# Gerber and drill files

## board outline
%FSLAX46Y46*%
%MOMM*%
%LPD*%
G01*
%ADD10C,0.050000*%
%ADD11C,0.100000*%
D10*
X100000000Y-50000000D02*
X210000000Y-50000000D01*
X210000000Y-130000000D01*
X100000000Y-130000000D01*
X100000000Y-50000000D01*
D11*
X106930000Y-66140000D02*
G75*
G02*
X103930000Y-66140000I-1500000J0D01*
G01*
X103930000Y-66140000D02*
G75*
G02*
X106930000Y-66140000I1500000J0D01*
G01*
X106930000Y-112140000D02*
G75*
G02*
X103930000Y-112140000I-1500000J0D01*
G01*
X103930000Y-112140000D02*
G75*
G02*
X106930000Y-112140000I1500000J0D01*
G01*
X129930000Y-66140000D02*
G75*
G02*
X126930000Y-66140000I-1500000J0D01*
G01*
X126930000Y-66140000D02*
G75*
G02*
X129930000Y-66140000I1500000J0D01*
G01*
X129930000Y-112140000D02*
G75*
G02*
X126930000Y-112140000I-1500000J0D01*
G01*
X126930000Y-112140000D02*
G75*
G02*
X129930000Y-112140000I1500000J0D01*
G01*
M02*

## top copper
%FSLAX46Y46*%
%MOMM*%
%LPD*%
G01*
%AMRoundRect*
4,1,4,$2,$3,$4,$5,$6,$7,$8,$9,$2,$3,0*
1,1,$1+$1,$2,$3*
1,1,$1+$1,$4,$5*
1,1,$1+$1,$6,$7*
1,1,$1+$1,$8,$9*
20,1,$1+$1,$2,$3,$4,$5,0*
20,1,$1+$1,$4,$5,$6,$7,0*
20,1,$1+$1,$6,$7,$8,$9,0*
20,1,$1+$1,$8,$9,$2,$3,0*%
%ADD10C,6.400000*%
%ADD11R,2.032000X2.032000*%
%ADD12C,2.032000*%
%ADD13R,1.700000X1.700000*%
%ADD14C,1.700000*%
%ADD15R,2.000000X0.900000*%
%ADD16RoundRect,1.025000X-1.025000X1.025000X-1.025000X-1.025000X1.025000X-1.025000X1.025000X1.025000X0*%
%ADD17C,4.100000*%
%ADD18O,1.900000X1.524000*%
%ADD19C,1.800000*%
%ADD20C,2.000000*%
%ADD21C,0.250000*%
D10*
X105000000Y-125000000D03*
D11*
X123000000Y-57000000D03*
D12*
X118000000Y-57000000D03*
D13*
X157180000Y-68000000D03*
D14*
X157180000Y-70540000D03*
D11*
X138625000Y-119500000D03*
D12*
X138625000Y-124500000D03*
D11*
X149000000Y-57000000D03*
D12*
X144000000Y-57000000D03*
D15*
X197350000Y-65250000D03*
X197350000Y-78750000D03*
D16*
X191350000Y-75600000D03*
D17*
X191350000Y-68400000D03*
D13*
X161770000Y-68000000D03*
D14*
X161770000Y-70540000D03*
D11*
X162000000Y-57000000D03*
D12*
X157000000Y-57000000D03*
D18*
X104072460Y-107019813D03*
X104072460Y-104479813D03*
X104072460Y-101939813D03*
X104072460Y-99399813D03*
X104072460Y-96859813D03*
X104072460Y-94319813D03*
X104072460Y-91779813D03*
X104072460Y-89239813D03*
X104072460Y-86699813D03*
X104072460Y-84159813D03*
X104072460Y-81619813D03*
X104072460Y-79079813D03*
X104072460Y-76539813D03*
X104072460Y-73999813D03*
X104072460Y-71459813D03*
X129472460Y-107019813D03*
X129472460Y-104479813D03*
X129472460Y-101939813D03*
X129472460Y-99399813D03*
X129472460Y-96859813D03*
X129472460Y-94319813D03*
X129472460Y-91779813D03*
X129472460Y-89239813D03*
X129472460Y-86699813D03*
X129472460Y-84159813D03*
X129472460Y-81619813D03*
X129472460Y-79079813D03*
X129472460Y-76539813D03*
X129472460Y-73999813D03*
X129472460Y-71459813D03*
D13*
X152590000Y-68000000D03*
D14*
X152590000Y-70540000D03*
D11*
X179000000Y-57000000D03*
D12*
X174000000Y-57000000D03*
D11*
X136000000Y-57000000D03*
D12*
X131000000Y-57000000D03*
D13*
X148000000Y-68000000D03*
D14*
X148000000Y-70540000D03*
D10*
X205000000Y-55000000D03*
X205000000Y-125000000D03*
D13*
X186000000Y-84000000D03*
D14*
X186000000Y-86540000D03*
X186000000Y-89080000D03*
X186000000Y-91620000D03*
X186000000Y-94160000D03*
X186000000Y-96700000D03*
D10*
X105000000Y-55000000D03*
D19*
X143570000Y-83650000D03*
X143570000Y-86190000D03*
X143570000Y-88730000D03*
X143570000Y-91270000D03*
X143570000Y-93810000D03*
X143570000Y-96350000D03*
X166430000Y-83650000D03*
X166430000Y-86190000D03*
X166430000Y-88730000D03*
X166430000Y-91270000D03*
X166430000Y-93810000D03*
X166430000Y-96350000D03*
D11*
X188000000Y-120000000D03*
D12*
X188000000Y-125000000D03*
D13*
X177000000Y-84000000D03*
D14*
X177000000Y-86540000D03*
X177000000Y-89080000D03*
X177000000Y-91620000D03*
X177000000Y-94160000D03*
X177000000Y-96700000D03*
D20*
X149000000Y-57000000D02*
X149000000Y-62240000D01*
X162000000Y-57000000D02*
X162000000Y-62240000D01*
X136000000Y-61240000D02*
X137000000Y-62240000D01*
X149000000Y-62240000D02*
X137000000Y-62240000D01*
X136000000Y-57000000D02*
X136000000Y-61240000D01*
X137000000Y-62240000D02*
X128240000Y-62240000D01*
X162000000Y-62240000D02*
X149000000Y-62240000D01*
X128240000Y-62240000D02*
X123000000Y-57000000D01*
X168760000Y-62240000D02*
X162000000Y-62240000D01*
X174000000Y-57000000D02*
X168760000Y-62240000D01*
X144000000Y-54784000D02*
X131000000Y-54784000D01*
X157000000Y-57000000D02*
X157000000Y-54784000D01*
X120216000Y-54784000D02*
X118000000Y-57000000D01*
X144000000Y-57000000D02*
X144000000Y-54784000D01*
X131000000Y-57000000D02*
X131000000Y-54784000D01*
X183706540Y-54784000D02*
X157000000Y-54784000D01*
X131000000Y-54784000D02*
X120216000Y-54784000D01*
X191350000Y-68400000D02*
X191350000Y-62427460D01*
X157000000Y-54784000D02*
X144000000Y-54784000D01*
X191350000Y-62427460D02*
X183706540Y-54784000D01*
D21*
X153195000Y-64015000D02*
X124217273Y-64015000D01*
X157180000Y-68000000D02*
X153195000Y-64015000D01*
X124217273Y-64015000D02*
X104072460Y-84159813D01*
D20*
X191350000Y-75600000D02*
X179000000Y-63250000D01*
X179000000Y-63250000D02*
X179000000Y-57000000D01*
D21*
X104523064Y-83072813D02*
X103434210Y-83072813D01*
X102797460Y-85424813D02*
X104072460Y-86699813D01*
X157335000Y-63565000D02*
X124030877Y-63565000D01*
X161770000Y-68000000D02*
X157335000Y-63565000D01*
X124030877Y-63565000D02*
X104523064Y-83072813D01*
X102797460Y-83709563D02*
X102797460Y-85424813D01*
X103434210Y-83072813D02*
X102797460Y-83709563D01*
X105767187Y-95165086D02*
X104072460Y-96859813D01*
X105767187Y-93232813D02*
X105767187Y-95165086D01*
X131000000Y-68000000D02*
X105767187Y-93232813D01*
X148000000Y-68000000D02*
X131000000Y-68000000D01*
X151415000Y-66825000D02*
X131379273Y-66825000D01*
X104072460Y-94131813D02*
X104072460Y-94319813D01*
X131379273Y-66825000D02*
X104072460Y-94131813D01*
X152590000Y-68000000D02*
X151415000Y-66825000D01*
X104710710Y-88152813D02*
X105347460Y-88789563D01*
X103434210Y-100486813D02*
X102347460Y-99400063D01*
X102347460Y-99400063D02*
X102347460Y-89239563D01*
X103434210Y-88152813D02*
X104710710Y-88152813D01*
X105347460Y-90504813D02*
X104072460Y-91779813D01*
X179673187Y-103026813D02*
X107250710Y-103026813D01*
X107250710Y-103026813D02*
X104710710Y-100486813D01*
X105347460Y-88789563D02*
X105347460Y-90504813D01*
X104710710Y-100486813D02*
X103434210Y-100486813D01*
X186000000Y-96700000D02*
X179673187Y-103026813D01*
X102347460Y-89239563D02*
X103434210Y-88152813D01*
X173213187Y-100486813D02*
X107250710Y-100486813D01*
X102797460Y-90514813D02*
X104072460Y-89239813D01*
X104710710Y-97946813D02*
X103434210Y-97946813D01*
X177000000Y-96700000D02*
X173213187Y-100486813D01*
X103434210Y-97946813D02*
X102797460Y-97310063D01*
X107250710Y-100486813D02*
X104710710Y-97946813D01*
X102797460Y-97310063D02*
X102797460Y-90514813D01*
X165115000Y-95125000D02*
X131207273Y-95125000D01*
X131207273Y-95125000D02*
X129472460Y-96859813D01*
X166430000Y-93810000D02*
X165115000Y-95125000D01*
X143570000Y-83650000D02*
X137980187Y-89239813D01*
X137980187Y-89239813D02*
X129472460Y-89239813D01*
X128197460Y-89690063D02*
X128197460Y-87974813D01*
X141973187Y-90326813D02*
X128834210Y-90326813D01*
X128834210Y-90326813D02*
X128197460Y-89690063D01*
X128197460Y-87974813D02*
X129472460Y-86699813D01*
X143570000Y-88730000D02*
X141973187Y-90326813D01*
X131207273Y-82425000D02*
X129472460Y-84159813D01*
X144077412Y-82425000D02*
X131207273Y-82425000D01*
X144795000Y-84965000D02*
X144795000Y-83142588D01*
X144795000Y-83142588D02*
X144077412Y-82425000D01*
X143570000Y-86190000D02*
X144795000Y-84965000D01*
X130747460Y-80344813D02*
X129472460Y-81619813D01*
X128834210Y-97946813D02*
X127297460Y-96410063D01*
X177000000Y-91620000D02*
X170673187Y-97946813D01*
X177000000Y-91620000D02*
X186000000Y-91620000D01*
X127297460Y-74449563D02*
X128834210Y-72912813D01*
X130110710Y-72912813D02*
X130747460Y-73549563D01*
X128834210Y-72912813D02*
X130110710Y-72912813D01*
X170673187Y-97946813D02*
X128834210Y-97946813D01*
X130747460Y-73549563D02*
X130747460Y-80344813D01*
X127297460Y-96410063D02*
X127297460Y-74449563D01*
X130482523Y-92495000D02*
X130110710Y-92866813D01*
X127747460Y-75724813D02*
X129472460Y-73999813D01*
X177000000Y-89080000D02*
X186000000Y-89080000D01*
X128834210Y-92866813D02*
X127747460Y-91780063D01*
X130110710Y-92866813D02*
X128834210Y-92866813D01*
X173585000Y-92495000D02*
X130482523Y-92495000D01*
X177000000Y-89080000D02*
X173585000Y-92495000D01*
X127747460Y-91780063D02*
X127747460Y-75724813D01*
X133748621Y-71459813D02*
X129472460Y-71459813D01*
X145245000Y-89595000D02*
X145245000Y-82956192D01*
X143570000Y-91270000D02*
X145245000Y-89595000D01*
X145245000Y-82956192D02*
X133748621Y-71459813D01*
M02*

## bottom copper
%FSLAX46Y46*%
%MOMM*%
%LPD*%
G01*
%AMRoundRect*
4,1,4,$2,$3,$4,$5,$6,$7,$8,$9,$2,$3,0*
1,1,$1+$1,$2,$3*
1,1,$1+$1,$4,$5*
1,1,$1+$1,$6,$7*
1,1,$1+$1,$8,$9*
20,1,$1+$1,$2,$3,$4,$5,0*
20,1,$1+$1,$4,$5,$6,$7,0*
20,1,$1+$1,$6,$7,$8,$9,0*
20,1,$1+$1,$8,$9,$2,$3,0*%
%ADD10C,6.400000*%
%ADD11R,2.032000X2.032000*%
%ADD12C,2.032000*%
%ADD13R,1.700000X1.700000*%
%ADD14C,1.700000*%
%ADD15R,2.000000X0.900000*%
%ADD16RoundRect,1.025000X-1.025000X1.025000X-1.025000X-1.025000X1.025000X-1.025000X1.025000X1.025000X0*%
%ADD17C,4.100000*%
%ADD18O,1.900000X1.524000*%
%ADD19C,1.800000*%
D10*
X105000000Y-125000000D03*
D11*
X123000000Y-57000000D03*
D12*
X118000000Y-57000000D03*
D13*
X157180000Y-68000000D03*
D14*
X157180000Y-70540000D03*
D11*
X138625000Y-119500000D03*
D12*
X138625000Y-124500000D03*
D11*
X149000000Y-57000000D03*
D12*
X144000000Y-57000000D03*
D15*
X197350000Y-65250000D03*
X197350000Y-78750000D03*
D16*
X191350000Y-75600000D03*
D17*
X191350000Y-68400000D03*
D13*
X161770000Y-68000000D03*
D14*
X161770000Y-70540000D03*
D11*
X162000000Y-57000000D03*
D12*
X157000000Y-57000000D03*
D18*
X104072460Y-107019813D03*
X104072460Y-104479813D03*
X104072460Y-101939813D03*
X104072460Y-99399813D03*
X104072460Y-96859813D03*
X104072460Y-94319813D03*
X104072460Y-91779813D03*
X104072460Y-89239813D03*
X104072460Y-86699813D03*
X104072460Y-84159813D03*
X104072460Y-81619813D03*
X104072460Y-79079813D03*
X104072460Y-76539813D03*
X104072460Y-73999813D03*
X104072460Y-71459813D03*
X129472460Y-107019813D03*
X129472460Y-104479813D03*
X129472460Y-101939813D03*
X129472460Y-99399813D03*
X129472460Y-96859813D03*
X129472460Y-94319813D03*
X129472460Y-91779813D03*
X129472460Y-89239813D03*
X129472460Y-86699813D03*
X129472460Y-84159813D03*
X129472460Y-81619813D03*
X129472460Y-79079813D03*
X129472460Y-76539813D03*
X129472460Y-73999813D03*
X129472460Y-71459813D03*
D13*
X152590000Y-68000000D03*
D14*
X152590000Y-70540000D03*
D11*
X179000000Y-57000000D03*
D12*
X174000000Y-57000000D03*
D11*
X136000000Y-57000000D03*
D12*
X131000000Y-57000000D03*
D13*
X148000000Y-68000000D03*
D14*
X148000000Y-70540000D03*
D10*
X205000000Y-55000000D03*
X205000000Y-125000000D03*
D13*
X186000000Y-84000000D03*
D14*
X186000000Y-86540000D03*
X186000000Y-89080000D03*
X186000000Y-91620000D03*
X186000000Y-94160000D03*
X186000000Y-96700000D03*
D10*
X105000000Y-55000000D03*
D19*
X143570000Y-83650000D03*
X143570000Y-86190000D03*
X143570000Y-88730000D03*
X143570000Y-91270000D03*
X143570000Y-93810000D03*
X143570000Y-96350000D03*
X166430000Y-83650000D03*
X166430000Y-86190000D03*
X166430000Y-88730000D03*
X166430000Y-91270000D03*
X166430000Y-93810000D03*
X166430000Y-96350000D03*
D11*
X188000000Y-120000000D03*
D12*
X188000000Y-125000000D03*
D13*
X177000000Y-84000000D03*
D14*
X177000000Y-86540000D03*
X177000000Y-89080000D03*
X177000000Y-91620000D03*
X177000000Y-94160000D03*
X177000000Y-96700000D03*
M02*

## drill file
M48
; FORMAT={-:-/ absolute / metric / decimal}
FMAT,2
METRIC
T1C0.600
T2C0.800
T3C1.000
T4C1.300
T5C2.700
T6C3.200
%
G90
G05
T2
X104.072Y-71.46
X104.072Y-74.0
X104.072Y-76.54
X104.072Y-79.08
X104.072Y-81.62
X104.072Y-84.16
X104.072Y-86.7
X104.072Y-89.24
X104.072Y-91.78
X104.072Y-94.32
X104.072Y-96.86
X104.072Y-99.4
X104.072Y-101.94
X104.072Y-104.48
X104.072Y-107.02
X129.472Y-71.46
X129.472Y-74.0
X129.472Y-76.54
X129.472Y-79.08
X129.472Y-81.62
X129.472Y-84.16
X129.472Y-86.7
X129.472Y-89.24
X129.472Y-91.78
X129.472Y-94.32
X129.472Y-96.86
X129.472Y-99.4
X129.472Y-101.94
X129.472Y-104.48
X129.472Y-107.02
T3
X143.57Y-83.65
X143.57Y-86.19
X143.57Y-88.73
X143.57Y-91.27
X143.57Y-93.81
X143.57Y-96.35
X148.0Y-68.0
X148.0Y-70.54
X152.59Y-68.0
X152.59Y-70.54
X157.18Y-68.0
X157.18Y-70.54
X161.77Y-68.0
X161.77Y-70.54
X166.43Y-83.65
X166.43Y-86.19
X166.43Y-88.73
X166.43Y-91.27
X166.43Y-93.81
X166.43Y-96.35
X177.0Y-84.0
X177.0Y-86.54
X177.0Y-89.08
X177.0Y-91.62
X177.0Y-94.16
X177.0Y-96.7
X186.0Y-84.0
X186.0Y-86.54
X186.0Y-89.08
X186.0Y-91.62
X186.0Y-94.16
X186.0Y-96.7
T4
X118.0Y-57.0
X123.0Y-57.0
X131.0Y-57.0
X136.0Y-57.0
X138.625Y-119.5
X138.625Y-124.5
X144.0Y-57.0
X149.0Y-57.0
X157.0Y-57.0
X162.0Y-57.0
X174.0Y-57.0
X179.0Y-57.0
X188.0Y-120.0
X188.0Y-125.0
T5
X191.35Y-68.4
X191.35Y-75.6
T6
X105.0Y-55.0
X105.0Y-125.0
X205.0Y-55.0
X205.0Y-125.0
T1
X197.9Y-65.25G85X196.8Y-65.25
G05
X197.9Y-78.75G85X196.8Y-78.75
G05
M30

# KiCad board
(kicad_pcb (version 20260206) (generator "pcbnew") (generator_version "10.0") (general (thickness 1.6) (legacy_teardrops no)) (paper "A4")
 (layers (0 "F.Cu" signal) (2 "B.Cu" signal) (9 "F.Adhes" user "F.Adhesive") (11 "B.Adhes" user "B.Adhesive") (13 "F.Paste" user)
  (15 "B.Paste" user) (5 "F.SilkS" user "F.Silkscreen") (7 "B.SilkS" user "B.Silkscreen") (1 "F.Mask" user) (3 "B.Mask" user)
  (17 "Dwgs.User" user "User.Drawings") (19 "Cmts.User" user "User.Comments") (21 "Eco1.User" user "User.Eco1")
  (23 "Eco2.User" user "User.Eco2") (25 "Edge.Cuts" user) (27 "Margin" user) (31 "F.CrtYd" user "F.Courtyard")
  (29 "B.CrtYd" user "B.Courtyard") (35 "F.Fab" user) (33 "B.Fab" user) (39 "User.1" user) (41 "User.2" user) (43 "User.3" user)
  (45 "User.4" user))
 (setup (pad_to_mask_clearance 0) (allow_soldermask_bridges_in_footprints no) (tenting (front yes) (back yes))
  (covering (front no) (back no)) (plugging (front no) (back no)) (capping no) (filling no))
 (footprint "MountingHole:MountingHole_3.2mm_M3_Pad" (layer "F.Cu") (at 105 125)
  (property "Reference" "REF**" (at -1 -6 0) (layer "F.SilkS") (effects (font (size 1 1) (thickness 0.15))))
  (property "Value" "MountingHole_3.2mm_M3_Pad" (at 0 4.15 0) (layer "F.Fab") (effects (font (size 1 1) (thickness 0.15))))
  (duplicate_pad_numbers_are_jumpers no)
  (pad "1" thru_hole circle (at 0 0) (size 6.4 6.4) (drill 3.2) (layers "*.Cu" "*.Mask") (remove_unused_layers no) (zone_connect 2)))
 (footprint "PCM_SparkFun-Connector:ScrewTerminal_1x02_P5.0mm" (layer "F.Cu") (at 123 57 180)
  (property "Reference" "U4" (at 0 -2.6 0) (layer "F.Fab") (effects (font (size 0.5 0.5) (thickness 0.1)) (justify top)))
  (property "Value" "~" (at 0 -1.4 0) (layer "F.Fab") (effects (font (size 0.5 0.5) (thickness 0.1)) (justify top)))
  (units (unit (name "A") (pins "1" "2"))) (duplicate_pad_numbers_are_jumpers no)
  (pad "1" thru_hole rect (at 0 0 180) (size 2.032 2.032) (drill 1.3) (layers "*.Cu" "*.Mask") (remove_unused_layers no) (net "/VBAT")
   (thermal_bridge_angle 0))
  (pad "2" thru_hole circle (at 5 0 180) (size 2.032 2.032) (drill 1.3) (layers "*.Cu" "*.Mask") (remove_unused_layers no) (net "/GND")))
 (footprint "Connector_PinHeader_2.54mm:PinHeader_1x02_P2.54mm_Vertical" (layer "F.Cu") (at 157.18 68)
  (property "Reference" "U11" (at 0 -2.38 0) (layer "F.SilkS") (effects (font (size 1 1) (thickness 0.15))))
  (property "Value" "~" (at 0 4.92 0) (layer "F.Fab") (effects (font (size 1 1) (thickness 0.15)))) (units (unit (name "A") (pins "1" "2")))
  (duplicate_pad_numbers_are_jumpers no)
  (pad "1" thru_hole rect (at 0 0) (size 1.7 1.7) (drill 1) (layers "*.Cu" "*.Mask") (remove_unused_layers no) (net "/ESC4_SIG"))
  (pad "2" thru_hole circle (at 0 2.54) (size 1.7 1.7) (drill 1) (layers "*.Cu" "*.Mask") (remove_unused_layers no) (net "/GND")))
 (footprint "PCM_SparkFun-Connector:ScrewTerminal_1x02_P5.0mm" (layer "F.Cu") (at 138.625 119.5 -90)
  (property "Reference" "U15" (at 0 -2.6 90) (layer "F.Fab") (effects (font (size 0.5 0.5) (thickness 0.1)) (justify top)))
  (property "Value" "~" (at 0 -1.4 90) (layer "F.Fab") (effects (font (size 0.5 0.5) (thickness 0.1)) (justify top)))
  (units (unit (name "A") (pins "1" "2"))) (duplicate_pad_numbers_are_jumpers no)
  (pad "1" thru_hole rect (at 0 0 270) (size 2.032 2.032) (drill 1.3) (layers "*.Cu" "*.Mask") (remove_unused_layers no)
   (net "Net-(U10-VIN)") (thermal_bridge_angle 0))
  (pad "2" thru_hole circle (at 5 0 270) (size 2.032 2.032) (drill 1.3) (layers "*.Cu" "*.Mask") (remove_unused_layers no)
   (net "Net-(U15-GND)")))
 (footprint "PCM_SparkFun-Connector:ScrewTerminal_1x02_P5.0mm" (layer "F.Cu") (at 149 57 180)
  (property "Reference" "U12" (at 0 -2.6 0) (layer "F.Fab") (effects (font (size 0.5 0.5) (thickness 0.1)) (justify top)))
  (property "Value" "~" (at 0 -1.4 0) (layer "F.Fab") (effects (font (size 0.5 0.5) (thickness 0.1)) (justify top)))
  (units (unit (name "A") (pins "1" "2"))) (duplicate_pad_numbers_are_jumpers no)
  (pad "1" thru_hole rect (at 0 0 180) (size 2.032 2.032) (drill 1.3) (layers "*.Cu" "*.Mask") (remove_unused_layers no) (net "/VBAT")
   (thermal_bridge_angle 0))
  (pad "2" thru_hole circle (at 5 0 180) (size 2.032 2.032) (drill 1.3) (layers "*.Cu" "*.Mask") (remove_unused_layers no) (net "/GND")))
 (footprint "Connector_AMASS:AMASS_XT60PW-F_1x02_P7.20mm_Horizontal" (layer "F.Cu") (at 191.35 75.6 -90)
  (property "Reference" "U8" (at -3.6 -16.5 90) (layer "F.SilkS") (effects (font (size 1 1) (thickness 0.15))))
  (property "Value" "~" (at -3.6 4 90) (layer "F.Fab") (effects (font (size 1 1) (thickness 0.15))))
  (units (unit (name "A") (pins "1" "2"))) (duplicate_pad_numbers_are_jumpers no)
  (pad "" thru_hole rect (at -10.35 -6 270) (size 0.9 2) (drill oval 0.6 1.7) (layers "*.Cu" "*.Mask") (remove_unused_layers no))
  (pad "" thru_hole rect (at 3.15 -6 270) (size 0.9 2) (drill oval 0.6 1.7) (layers "*.Cu" "*.Mask") (remove_unused_layers no))
  (pad "1" thru_hole roundrect (at 0 0 270) (size 4.1 4.1) (drill 2.7) (layers "*.Cu" "*.Mask") (remove_unused_layers no)
   (roundrect_rratio 0.25) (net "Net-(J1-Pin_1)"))
  (pad "2" thru_hole circle (at -7.2 0 270) (size 4.1 4.1) (drill 2.7) (layers "*.Cu" "*.Mask") (remove_unused_layers no) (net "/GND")))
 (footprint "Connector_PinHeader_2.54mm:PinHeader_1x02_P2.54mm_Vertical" (layer "F.Cu") (at 161.77 68)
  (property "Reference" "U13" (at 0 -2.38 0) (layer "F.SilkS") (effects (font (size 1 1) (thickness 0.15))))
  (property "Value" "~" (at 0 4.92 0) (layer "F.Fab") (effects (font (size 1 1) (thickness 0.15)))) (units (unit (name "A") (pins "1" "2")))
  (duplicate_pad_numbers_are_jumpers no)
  (pad "1" thru_hole rect (at 0 0) (size 1.7 1.7) (drill 1) (layers "*.Cu" "*.Mask") (remove_unused_layers no) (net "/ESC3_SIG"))
  (pad "2" thru_hole circle (at 0 2.54) (size 1.7 1.7) (drill 1) (layers "*.Cu" "*.Mask") (remove_unused_layers no) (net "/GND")))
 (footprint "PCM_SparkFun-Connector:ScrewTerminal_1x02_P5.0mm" (layer "F.Cu") (at 162 57 180)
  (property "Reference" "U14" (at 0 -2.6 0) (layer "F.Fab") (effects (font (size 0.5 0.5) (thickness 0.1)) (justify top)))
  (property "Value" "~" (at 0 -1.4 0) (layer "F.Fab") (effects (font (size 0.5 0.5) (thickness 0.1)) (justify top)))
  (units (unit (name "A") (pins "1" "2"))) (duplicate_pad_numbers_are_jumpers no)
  (pad "1" thru_hole rect (at 0 0 180) (size 2.032 2.032) (drill 1.3) (layers "*.Cu" "*.Mask") (remove_unused_layers no) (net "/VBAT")
   (thermal_bridge_angle 0))
  (pad "2" thru_hole circle (at 5 0 180) (size 2.032 2.032) (drill 1.3) (layers "*.Cu" "*.Mask") (remove_unused_layers no) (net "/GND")))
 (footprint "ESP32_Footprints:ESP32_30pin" (layer "F.Cu") (at 116 90)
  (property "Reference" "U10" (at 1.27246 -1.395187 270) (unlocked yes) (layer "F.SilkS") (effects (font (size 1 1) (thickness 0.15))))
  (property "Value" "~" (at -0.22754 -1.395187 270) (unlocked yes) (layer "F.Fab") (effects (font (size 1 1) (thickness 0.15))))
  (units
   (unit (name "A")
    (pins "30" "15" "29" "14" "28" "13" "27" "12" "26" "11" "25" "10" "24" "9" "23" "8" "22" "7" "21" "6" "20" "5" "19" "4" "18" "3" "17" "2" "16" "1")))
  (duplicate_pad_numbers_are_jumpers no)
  (fp_circle (center -10.57 -23.86) (end -10.57 -22.36) (stroke (width 0.1) (type default)) (fill no) (layer "Edge.Cuts"))
  (fp_circle (center -10.57 22.14) (end -10.57 23.64) (stroke (width 0.1) (type default)) (fill no) (layer "Edge.Cuts"))
  (fp_circle (center 12.43 -23.86) (end 12.43 -22.36) (stroke (width 0.1) (type default)) (fill no) (layer "Edge.Cuts"))
  (fp_circle (center 12.43 22.14) (end 12.43 23.64) (stroke (width 0.1) (type default)) (fill no) (layer "Edge.Cuts"))
  (pad "1" thru_hole oval (at -11.92754 17.019813 270) (size 1.524 1.9) (drill 0.8) (layers "*.Cu" "*.Mask") (remove_unused_layers no)
   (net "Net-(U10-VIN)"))
  (pad "2" thru_hole oval (at -11.92754 14.479813 270) (size 1.524 1.9) (drill 0.8) (layers "*.Cu" "*.Mask") (remove_unused_layers no)
   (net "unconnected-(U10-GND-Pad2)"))
  (pad "3" thru_hole oval (at -11.92754 11.939813 270) (size 1.524 1.9) (drill 0.8) (layers "*.Cu" "*.Mask") (remove_unused_layers no)
   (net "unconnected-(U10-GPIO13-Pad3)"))
  (pad "4" thru_hole oval (at -11.92754 9.399813 270) (size 1.524 1.9) (drill 0.8) (layers "*.Cu" "*.Mask") (remove_unused_layers no)
   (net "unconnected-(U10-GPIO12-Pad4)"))
  (pad "5" thru_hole oval (at -11.92754 6.859813 270) (size 1.524 1.9) (drill 0.8) (layers "*.Cu" "*.Mask") (remove_unused_layers no)
   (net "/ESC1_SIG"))
  (pad "6" thru_hole oval (at -11.92754 4.319813 270) (size 1.524 1.9) (drill 0.8) (layers "*.Cu" "*.Mask") (remove_unused_layers no)
   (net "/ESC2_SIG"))
  (pad "7" thru_hole oval (at -11.92754 1.779813 270) (size 1.524 1.9) (drill 0.8) (layers "*.Cu" "*.Mask") (remove_unused_layers no)
   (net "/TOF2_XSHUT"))
  (pad "8" thru_hole oval (at -11.92754 -0.760187 270) (size 1.524 1.9) (drill 0.8) (layers "*.Cu" "*.Mask") (remove_unused_layers no)
   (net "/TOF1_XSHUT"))
  (pad "9" thru_hole oval (at -11.92754 -3.300187 270) (size 1.524 1.9) (drill 0.8) (layers "*.Cu" "*.Mask") (remove_unused_layers no)
   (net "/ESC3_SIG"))
  (pad "10" thru_hole oval (at -11.92754 -5.840187 270) (size 1.524 1.9) (drill 0.8) (layers "*.Cu" "*.Mask") (remove_unused_layers no)
   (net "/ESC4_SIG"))
  (pad "11" thru_hole oval (at -11.92754 -8.380187 270) (size 1.524 1.9) (drill 0.8) (layers "*.Cu" "*.Mask") (remove_unused_layers no)
   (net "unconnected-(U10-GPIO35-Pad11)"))
  (pad "12" thru_hole oval (at -11.92754 -10.920187 270) (size 1.524 1.9) (drill 0.8) (layers "*.Cu" "*.Mask") (remove_unused_layers no)
   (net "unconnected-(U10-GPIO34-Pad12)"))
  (pad "13" thru_hole oval (at -11.92754 -13.460187 270) (size 1.524 1.9) (drill 0.8) (layers "*.Cu" "*.Mask") (remove_unused_layers no)
   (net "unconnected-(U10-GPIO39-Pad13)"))
  (pad "14" thru_hole oval (at -11.92754 -16.000187 270) (size 1.524 1.9) (drill 0.8) (layers "*.Cu" "*.Mask") (remove_unused_layers no)
   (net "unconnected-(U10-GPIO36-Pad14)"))
  (pad "15" thru_hole oval (at -11.92754 -18.540187 270) (size 1.524 1.9) (drill 0.8) (layers "*.Cu" "*.Mask") (remove_unused_layers no)
   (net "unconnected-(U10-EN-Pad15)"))
  (pad "16" thru_hole oval (at 13.47246 17.019813 270) (size 1.524 1.9) (drill 0.8) (layers "*.Cu" "*.Mask") (remove_unused_layers no)
   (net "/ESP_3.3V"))
  (pad "17" thru_hole oval (at 13.47246 14.479813 270) (size 1.524 1.9) (drill 0.8) (layers "*.Cu" "*.Mask") (remove_unused_layers no)
   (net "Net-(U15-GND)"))
  (pad "18" thru_hole oval (at 13.47246 11.939813 270) (size 1.524 1.9) (drill 0.8) (layers "*.Cu" "*.Mask") (remove_unused_layers no)
   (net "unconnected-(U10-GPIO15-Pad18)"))
  (pad "19" thru_hole oval (at 13.47246 9.399813 270) (size 1.524 1.9) (drill 0.8) (layers "*.Cu" "*.Mask") (remove_unused_layers no)
   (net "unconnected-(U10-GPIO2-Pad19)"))
  (pad "20" thru_hole oval (at 13.47246 6.859813 270) (size 1.524 1.9) (drill 0.8) (layers "*.Cu" "*.Mask" "Dwgs.User")
   (remove_unused_layers no) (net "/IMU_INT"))
  (pad "21" thru_hole oval (at 13.47246 4.319813 270) (size 1.524 1.9) (drill 0.8) (layers "*.Cu" "*.Mask") (remove_unused_layers no)
   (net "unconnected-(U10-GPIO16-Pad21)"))
  (pad "22" thru_hole oval (at 13.47246 1.779813 270) (size 1.524 1.9) (drill 0.8) (layers "*.Cu" "*.Mask") (remove_unused_layers no)
   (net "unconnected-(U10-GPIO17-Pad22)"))
  (pad "23" thru_hole oval (at 13.47246 -0.760187 270) (size 1.524 1.9) (drill 0.8) (layers "*.Cu" "*.Mask") (remove_unused_layers no)
   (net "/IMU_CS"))
  (pad "24" thru_hole oval (at 13.47246 -3.300187 270) (size 1.524 1.9) (drill 0.8) (layers "*.Cu" "*.Mask") (remove_unused_layers no)
   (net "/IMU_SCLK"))
  (pad "25" thru_hole oval (at 13.47246 -5.840187 270) (size 1.524 1.9) (drill 0.8) (layers "*.Cu" "*.Mask") (remove_unused_layers no)
   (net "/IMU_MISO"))
  (pad "26" thru_hole oval (at 13.47246 -8.380187 270) (size 1.524 1.9) (drill 0.8) (layers "*.Cu" "*.Mask") (remove_unused_layers no)
   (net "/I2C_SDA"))
  (pad "27" thru_hole oval (at 13.47246 -10.920187 270) (size 1.524 1.9) (drill 0.8) (layers "*.Cu" "*.Mask") (remove_unused_layers no)
   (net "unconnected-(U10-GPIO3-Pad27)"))
  (pad "28" thru_hole oval (at 13.47246 -13.460187 270) (size 1.524 1.9) (drill 0.8) (layers "*.Cu" "*.Mask") (remove_unused_layers no)
   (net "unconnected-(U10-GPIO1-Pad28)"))
  (pad "29" thru_hole oval (at 13.47246 -16.000187 270) (size 1.524 1.9) (drill 0.8) (layers "*.Cu" "*.Mask") (remove_unused_layers no)
   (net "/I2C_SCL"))
  (pad "30" thru_hole oval (at 13.47246 -18.540187 270) (size 1.524 1.9) (drill 0.8) (layers "*.Cu" "*.Mask") (remove_unused_layers no)
   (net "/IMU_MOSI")))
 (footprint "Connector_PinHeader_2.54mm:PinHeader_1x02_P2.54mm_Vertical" (layer "F.Cu") (at 152.59 68)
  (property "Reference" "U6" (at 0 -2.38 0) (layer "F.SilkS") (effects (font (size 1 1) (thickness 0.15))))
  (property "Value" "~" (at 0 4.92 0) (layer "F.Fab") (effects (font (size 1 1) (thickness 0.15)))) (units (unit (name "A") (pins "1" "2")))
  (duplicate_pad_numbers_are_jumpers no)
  (pad "1" thru_hole rect (at 0 0) (size 1.7 1.7) (drill 1) (layers "*.Cu" "*.Mask") (remove_unused_layers no) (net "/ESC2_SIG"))
  (pad "2" thru_hole circle (at 0 2.54) (size 1.7 1.7) (drill 1) (layers "*.Cu" "*.Mask") (remove_unused_layers no) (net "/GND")))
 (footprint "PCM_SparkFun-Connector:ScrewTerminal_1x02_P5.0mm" (layer "F.Cu") (at 179 57 180)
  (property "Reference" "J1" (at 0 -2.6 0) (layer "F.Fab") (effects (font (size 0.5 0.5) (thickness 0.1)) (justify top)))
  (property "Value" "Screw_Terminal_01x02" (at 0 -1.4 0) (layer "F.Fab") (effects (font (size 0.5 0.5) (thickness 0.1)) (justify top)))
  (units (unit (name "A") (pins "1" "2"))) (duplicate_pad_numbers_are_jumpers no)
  (pad "1" thru_hole rect (at 0 0 180) (size 2.032 2.032) (drill 1.3) (layers "*.Cu" "*.Mask") (remove_unused_layers no)
   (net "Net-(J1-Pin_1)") (thermal_bridge_angle 0))
  (pad "2" thru_hole circle (at 5 0 180) (size 2.032 2.032) (drill 1.3) (layers "*.Cu" "*.Mask") (remove_unused_layers no) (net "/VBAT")))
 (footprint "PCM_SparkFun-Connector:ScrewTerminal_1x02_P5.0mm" (layer "F.Cu") (at 136 57 180)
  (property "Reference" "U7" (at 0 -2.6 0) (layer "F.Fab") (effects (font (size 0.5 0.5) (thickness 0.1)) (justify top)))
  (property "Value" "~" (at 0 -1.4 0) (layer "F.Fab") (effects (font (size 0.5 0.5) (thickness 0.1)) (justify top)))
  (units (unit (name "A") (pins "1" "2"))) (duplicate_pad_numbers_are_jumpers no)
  (pad "1" thru_hole rect (at 0 0 180) (size 2.032 2.032) (drill 1.3) (layers "*.Cu" "*.Mask") (remove_unused_layers no) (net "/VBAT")
   (thermal_bridge_angle 0))
  (pad "2" thru_hole circle (at 5 0 180) (size 2.032 2.032) (drill 1.3) (layers "*.Cu" "*.Mask") (remove_unused_layers no) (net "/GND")))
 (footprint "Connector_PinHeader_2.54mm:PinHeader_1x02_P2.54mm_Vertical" (layer "F.Cu") (at 148 68)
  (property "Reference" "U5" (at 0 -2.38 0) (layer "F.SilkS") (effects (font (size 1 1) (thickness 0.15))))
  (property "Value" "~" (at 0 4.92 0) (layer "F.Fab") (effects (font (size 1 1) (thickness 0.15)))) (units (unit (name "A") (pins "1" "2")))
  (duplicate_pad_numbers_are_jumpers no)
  (pad "1" thru_hole rect (at 0 0) (size 1.7 1.7) (drill 1) (layers "*.Cu" "*.Mask") (remove_unused_layers no) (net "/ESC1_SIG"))
  (pad "2" thru_hole circle (at 0 2.54) (size 1.7 1.7) (drill 1) (layers "*.Cu" "*.Mask") (remove_unused_layers no) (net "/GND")))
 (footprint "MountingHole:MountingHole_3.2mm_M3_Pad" (layer "F.Cu") (at 205 55)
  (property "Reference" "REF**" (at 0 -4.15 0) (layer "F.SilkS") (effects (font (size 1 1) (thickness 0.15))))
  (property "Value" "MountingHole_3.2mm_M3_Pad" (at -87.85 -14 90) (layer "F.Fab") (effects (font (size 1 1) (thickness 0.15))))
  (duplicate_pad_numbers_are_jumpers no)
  (pad "1" thru_hole circle (at 0 0) (size 6.4 6.4) (drill 3.2) (layers "*.Cu" "*.Mask") (remove_unused_layers no) (zone_connect 2)))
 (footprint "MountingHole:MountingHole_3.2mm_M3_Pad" (layer "F.Cu") (at 205 125)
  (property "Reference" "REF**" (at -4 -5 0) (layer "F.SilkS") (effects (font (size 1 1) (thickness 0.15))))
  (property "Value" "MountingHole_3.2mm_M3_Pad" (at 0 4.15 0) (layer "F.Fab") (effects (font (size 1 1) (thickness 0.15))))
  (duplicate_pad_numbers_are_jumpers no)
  (pad "1" thru_hole circle (at 0 0) (size 6.4 6.4) (drill 3.2) (layers "*.Cu" "*.Mask") (remove_unused_layers no) (zone_connect 2)))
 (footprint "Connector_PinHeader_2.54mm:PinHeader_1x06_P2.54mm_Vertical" (layer "F.Cu") (at 186 84)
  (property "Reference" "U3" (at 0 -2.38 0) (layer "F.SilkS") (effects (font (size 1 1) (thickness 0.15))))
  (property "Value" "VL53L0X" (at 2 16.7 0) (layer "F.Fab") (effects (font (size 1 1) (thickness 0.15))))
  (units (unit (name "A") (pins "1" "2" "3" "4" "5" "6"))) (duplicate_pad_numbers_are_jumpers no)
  (pad "1" thru_hole rect (at 0 0) (size 1.7 1.7) (drill 1) (layers "*.Cu" "*.Mask") (remove_unused_layers no) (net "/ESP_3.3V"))
  (pad "2" thru_hole circle (at 0 2.54) (size 1.7 1.7) (drill 1) (layers "*.Cu" "*.Mask") (remove_unused_layers no) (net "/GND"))
  (pad "3" thru_hole circle (at 0 5.08) (size 1.7 1.7) (drill 1) (layers "*.Cu" "*.Mask") (remove_unused_layers no) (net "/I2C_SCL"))
  (pad "4" thru_hole circle (at 0 7.62) (size 1.7 1.7) (drill 1) (layers "*.Cu" "*.Mask") (remove_unused_layers no) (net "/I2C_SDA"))
  (pad "5" thru_hole circle (at 0 10.16) (size 1.7 1.7) (drill 1) (layers "*.Cu" "*.Mask") (remove_unused_layers no)
   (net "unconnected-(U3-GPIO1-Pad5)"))
  (pad "6" thru_hole circle (at 0 12.7) (size 1.7 1.7) (drill 1) (layers "*.Cu" "*.Mask") (remove_unused_layers no) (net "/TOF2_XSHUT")))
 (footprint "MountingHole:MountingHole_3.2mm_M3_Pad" (layer "F.Cu") (at 105 55)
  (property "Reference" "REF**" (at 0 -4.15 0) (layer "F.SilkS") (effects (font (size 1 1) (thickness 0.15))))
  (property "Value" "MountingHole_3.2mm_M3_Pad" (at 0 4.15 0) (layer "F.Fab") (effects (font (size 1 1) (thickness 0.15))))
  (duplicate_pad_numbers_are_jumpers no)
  (pad "1" thru_hole circle (at 0 0) (size 6.4 6.4) (drill 3.2) (layers "*.Cu" "*.Mask") (remove_unused_layers no) (zone_connect 2)))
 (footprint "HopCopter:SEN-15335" (layer "F.Cu") (at 143.57 83.65)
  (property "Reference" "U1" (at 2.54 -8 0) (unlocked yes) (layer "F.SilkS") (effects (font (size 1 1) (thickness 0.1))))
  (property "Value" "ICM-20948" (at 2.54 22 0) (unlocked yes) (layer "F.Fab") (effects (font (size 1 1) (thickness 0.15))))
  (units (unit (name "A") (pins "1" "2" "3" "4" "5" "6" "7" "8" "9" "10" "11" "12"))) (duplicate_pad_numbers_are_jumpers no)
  (pad "1" thru_hole circle (at 0 0) (size 1.8 1.8) (drill 1) (layers "*.Cu" "*.Mask") (remove_unused_layers no) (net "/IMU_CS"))
  (pad "2" thru_hole circle (at 0 2.54) (size 1.8 1.8) (drill 1) (layers "*.Cu" "*.Mask" "Eco1.User") (remove_unused_layers no)
   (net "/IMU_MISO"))
  (pad "3" thru_hole circle (at 0 5.08) (size 1.8 1.8) (drill 1) (layers "*.Cu" "*.Mask" "Eco1.User") (remove_unused_layers no)
   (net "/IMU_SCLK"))
  (pad "4" thru_hole circle (at 0 7.62) (size 1.8 1.8) (drill 1) (layers "*.Cu" "*.Mask" "Eco1.User") (remove_unused_layers no)
   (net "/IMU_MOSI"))
  (pad "5" thru_hole circle (at 0 10.16) (size 1.8 1.8) (drill 1) (layers "*.Cu" "*.Mask" "Eco1.User") (remove_unused_layers no)
   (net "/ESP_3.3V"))
  (pad "6" thru_hole circle (at 0 12.7) (size 1.8 1.8) (drill 1) (layers "*.Cu" "*.Mask" "Eco1.User") (remove_unused_layers no) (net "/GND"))
  (pad "7" thru_hole circle (at 22.86 0) (size 1.8 1.8) (drill 1) (layers "*.Cu" "*.Mask") (remove_unused_layers no)
   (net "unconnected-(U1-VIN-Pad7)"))
  (pad "8" thru_hole circle (at 22.86 2.54) (size 1.8 1.8) (drill 1) (layers "*.Cu" "*.Mask" "Eco1.User") (remove_unused_layers no)
   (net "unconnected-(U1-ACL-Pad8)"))
  (pad "9" thru_hole circle (at 22.86 5.08) (size 1.8 1.8) (drill 1) (layers "*.Cu" "*.Mask" "Eco1.User") (remove_unused_layers no)
   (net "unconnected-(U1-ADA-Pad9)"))
  (pad "10" thru_hole circle (at 22.86 7.62) (size 1.8 1.8) (drill 1) (layers "*.Cu" "*.Mask" "Eco1.User") (remove_unused_layers no)
   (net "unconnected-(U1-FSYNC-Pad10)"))
  (pad "11" thru_hole circle (at 22.86 10.16) (size 1.8 1.8) (drill 1) (layers "*.Cu" "*.Mask" "Eco1.User") (remove_unused_layers no)
   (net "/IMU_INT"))
  (pad "12" thru_hole circle (at 22.86 12.7) (size 1.8 1.8) (drill 1) (layers "*.Cu" "*.Mask" "Eco1.User") (remove_unused_layers no)
   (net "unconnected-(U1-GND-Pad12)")))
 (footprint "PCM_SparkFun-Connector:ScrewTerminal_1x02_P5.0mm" (layer "F.Cu") (at 188 120 -90)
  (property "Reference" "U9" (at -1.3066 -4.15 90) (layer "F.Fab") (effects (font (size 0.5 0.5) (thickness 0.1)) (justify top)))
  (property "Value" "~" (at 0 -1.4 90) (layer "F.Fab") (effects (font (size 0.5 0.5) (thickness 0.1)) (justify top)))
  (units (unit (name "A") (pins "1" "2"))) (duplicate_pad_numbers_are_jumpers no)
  (pad "1" thru_hole rect (at 0 0 270) (size 2.032 2.032) (drill 1.3) (layers "*.Cu" "*.Mask") (remove_unused_layers no) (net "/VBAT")
   (thermal_bridge_angle 0))
  (pad "2" thru_hole circle (at 5 0 270) (size 2.032 2.032) (drill 1.3) (layers "*.Cu" "*.Mask") (remove_unused_layers no) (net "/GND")))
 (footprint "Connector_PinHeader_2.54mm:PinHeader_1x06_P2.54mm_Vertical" (layer "F.Cu") (at 177 84)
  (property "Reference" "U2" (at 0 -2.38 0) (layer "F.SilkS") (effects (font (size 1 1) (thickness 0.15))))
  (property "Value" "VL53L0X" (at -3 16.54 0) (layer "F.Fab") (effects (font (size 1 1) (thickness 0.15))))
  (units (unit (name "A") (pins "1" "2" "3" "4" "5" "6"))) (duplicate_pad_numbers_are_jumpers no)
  (pad "1" thru_hole rect (at 0 0) (size 1.7 1.7) (drill 1) (layers "*.Cu" "*.Mask") (remove_unused_layers no) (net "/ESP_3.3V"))
  (pad "2" thru_hole circle (at 0 2.54) (size 1.7 1.7) (drill 1) (layers "*.Cu" "*.Mask") (remove_unused_layers no) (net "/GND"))
  (pad "3" thru_hole circle (at 0 5.08) (size 1.7 1.7) (drill 1) (layers "*.Cu" "*.Mask") (remove_unused_layers no) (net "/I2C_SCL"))
  (pad "4" thru_hole circle (at 0 7.62) (size 1.7 1.7) (drill 1) (layers "*.Cu" "*.Mask") (remove_unused_layers no) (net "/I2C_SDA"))
  (pad "5" thru_hole circle (at 0 10.16) (size 1.7 1.7) (drill 1) (layers "*.Cu" "*.Mask") (remove_unused_layers no)
   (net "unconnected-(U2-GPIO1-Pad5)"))
  (pad "6" thru_hole circle (at 0 12.7) (size 1.7 1.7) (drill 1) (layers "*.Cu" "*.Mask") (remove_unused_layers no) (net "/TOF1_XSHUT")))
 (gr_rect (start 100 50) (end 210 130) (stroke (width 0.05) (type solid)) (fill no) (layer "Edge.Cuts"))
 (segment (start 149 57) (end 149 62.24) (width 2) (layer "F.Cu") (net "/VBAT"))
 (segment (start 162 57) (end 162 62.24) (width 2) (layer "F.Cu") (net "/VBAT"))
 (segment (start 136 61.24) (end 137 62.24) (width 2) (layer "F.Cu") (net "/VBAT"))
 (segment (start 149 62.24) (end 137 62.24) (width 2) (layer "F.Cu") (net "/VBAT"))
 (segment (start 136 57) (end 136 61.24) (width 2) (layer "F.Cu") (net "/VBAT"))
 (segment (start 137 62.24) (end 128.24 62.24) (width 2) (layer "F.Cu") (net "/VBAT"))
 (segment (start 162 62.24) (end 149 62.24) (width 2) (layer "F.Cu") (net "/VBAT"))
 (segment (start 128.24 62.24) (end 123 57) (width 2) (layer "F.Cu") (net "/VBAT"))
 (segment (start 168.76 62.24) (end 162 62.24) (width 2) (layer "F.Cu") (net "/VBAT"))
 (segment (start 174 57) (end 168.76 62.24) (width 2) (layer "F.Cu") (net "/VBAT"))
 (segment (start 144 54.784) (end 131 54.784) (width 2) (layer "F.Cu") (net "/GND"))
 (segment (start 157 57) (end 157 54.784) (width 2) (layer "F.Cu") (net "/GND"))
 (segment (start 120.216 54.784) (end 118 57) (width 2) (layer "F.Cu") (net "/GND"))
 (segment (start 144 57) (end 144 54.784) (width 2) (layer "F.Cu") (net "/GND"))
 (segment (start 131 57) (end 131 54.784) (width 2) (layer "F.Cu") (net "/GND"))
 (segment (start 183.70654 54.784) (end 157 54.784) (width 2) (layer "F.Cu") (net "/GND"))
 (segment (start 131 54.784) (end 120.216 54.784) (width 2) (layer "F.Cu") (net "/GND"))
 (segment (start 191.35 68.4) (end 191.35 62.42746) (width 2) (layer "F.Cu") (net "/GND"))
 (segment (start 157 54.784) (end 144 54.784) (width 2) (layer "F.Cu") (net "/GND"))
 (segment (start 191.35 62.42746) (end 183.70654 54.784) (width 2) (layer "F.Cu") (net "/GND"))
 (segment (start 153.195 64.015) (end 124.217273 64.015) (width 0.25) (layer "F.Cu") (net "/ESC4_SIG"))
 (segment (start 157.18 68) (end 153.195 64.015) (width 0.25) (layer "F.Cu") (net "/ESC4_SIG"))
 (segment (start 124.217273 64.015) (end 104.07246 84.159813) (width 0.25) (layer "F.Cu") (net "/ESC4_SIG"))
 (segment (start 191.35 75.6) (end 179 63.25) (width 2) (layer "F.Cu") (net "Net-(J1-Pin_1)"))
 (segment (start 179 63.25) (end 179 57) (width 2) (layer "F.Cu") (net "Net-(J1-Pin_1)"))
 (segment (start 104.523064 83.072813) (end 103.43421 83.072813) (width 0.25) (layer "F.Cu") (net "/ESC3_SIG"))
 (segment (start 102.79746 85.424813) (end 104.07246 86.699813) (width 0.25) (layer "F.Cu") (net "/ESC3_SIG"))
 (segment (start 157.335 63.565) (end 124.030877 63.565) (width 0.25) (layer "F.Cu") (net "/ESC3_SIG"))
 (segment (start 161.77 68) (end 157.335 63.565) (width 0.25) (layer "F.Cu") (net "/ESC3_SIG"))
 (segment (start 124.030877 63.565) (end 104.523064 83.072813) (width 0.25) (layer "F.Cu") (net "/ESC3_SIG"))
 (segment (start 102.79746 83.709563) (end 102.79746 85.424813) (width 0.25) (layer "F.Cu") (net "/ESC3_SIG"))
 (segment (start 103.43421 83.072813) (end 102.79746 83.709563) (width 0.25) (layer "F.Cu") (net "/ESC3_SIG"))
 (segment (start 105.767187 95.165086) (end 104.07246 96.859813) (width 0.25) (layer "F.Cu") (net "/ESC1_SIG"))
 (segment (start 105.767187 93.232813) (end 105.767187 95.165086) (width 0.25) (layer "F.Cu") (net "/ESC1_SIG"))
 (segment (start 131 68) (end 105.767187 93.232813) (width 0.25) (layer "F.Cu") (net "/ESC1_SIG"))
 (segment (start 148 68) (end 131 68) (width 0.25) (layer "F.Cu") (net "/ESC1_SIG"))
 (segment (start 151.415 66.825) (end 131.379273 66.825) (width 0.25) (layer "F.Cu") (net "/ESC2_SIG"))
 (segment (start 104.07246 94.131813) (end 104.07246 94.319813) (width 0.25) (layer "F.Cu") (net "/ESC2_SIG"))
 (segment (start 131.379273 66.825) (end 104.07246 94.131813) (width 0.25) (layer "F.Cu") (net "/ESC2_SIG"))
 (segment (start 152.59 68) (end 151.415 66.825) (width 0.25) (layer "F.Cu") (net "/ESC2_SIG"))
 (segment (start 104.71071 88.152813) (end 105.34746 88.789563) (width 0.25) (layer "F.Cu") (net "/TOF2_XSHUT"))
 (segment (start 103.43421 100.486813) (end 102.34746 99.400063) (width 0.25) (layer "F.Cu") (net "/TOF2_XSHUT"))
 (segment (start 102.34746 99.400063) (end 102.34746 89.239563) (width 0.25) (layer "F.Cu") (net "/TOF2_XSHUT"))
 (segment (start 103.43421 88.152813) (end 104.71071 88.152813) (width 0.25) (layer "F.Cu") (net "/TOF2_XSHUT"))
 (segment (start 105.34746 90.504813) (end 104.07246 91.779813) (width 0.25) (layer "F.Cu") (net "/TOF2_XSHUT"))
 (segment (start 179.673187 103.026813) (end 107.25071 103.026813) (width 0.25) (layer "F.Cu") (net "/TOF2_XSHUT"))
 (segment (start 107.25071 103.026813) (end 104.71071 100.486813) (width 0.25) (layer "F.Cu") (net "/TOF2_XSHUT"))
 (segment (start 105.34746 88.789563) (end 105.34746 90.504813) (width 0.25) (layer "F.Cu") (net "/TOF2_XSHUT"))
 (segment (start 104.71071 100.486813) (end 103.43421 100.486813) (width 0.25) (layer "F.Cu") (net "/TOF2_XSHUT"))
 (segment (start 186 96.7) (end 179.673187 103.026813) (width 0.25) (layer "F.Cu") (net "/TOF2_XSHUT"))
 (segment (start 102.34746 89.239563) (end 103.43421 88.152813) (width 0.25) (layer "F.Cu") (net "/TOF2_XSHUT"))
 (segment (start 173.213187 100.486813) (end 107.25071 100.486813) (width 0.25) (layer "F.Cu") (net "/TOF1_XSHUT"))
 (segment (start 102.79746 90.514813) (end 104.07246 89.239813) (width 0.25) (layer "F.Cu") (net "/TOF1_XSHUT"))
 (segment (start 104.71071 97.946813) (end 103.43421 97.946813) (width 0.25) (layer "F.Cu") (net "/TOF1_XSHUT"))
 (segment (start 177 96.7) (end 173.213187 100.486813) (width 0.25) (layer "F.Cu") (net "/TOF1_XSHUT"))
 (segment (start 103.43421 97.946813) (end 102.79746 97.310063) (width 0.25) (layer "F.Cu") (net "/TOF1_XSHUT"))
 (segment (start 107.25071 100.486813) (end 104.71071 97.946813) (width 0.25) (layer "F.Cu") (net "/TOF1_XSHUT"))
 (segment (start 102.79746 97.310063) (end 102.79746 90.514813) (width 0.25) (layer "F.Cu") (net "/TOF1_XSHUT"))
 (segment (start 165.115 95.125) (end 131.207273 95.125) (width 0.25) (layer "F.Cu") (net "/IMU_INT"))
 (segment (start 131.207273 95.125) (end 129.47246 96.859813) (width 0.25) (layer "F.Cu") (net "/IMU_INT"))
 (segment (start 166.43 93.81) (end 165.115 95.125) (width 0.25) (layer "F.Cu") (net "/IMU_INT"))
 (segment (start 143.57 83.65) (end 137.980187 89.239813) (width 0.25) (layer "F.Cu") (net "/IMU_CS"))
 (segment (start 137.980187 89.239813) (end 129.47246 89.239813) (width 0.25) (layer "F.Cu") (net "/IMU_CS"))
 (segment (start 128.19746 89.690063) (end 128.19746 87.974813) (width 0.25) (layer "F.Cu") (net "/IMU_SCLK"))
 (segment (start 141.973187 90.326813) (end 128.83421 90.326813) (width 0.25) (layer "F.Cu") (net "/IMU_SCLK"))
 (segment (start 128.83421 90.326813) (end 128.19746 89.690063) (width 0.25) (layer "F.Cu") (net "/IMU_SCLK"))
 (segment (start 128.19746 87.974813) (end 129.47246 86.699813) (width 0.25) (layer "F.Cu") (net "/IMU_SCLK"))
 (segment (start 143.57 88.73) (end 141.973187 90.326813) (width 0.25) (layer "F.Cu") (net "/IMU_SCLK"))
 (segment (start 131.207273 82.425) (end 129.47246 84.159813) (width 0.25) (layer "F.Cu") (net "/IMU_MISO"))
 (segment (start 144.077412 82.425) (end 131.207273 82.425) (width 0.25) (layer "F.Cu") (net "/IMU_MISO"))
 (segment (start 144.795 84.965) (end 144.795 83.142588) (width 0.25) (layer "F.Cu") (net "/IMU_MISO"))
 (segment (start 144.795 83.142588) (end 144.077412 82.425) (width 0.25) (layer "F.Cu") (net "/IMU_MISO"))
 (segment (start 143.57 86.19) (end 144.795 84.965) (width 0.25) (layer "F.Cu") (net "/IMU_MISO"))
 (segment (start 130.74746 80.344813) (end 129.47246 81.619813) (width 0.25) (layer "F.Cu") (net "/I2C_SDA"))
 (segment (start 128.83421 97.946813) (end 127.29746 96.410063) (width 0.25) (layer "F.Cu") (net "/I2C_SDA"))
 (segment (start 177 91.62) (end 170.673187 97.946813) (width 0.25) (layer "F.Cu") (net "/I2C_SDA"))
 (segment (start 177 91.62) (end 186 91.62) (width 0.25) (layer "F.Cu") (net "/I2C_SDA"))
 (segment (start 127.29746 74.449563) (end 128.83421 72.912813) (width 0.25) (layer "F.Cu") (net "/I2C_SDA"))
 (segment (start 130.11071 72.912813) (end 130.74746 73.549563) (width 0.25) (layer "F.Cu") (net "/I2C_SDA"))
 (segment (start 128.83421 72.912813) (end 130.11071 72.912813) (width 0.25) (layer "F.Cu") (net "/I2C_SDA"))
 (segment (start 170.673187 97.946813) (end 128.83421 97.946813) (width 0.25) (layer "F.Cu") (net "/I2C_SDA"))
 (segment (start 130.74746 73.549563) (end 130.74746 80.344813) (width 0.25) (layer "F.Cu") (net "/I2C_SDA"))
 (segment (start 127.29746 96.410063) (end 127.29746 74.449563) (width 0.25) (layer "F.Cu") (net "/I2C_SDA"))
 (segment (start 130.482523 92.495) (end 130.11071 92.866813) (width 0.25) (layer "F.Cu") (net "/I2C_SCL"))
 (segment (start 127.74746 75.724813) (end 129.47246 73.999813) (width 0.25) (layer "F.Cu") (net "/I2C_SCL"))
 (segment (start 177 89.08) (end 186 89.08) (width 0.25) (layer "F.Cu") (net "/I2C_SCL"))
 (segment (start 128.83421 92.866813) (end 127.74746 91.780063) (width 0.25) (layer "F.Cu") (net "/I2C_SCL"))
 (segment (start 130.11071 92.866813) (end 128.83421 92.866813) (width 0.25) (layer "F.Cu") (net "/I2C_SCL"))
 (segment (start 173.585 92.495) (end 130.482523 92.495) (width 0.25) (layer "F.Cu") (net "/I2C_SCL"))
 (segment (start 177 89.08) (end 173.585 92.495) (width 0.25) (layer "F.Cu") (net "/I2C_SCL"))
 (segment (start 127.74746 91.780063) (end 127.74746 75.724813) (width 0.25) (layer "F.Cu") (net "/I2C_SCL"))
 (segment (start 133.748621 71.459813) (end 129.47246 71.459813) (width 0.25) (layer "F.Cu") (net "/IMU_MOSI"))
 (segment (start 145.245 89.595) (end 145.245 82.956192) (width 0.25) (layer "F.Cu") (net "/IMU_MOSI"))
 (segment (start 143.57 91.27) (end 145.245 89.595) (width 0.25) (layer "F.Cu") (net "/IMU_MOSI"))
 (segment (start 145.245 82.956192) (end 133.748621 71.459813) (width 0.25) (layer "F.Cu") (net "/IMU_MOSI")))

